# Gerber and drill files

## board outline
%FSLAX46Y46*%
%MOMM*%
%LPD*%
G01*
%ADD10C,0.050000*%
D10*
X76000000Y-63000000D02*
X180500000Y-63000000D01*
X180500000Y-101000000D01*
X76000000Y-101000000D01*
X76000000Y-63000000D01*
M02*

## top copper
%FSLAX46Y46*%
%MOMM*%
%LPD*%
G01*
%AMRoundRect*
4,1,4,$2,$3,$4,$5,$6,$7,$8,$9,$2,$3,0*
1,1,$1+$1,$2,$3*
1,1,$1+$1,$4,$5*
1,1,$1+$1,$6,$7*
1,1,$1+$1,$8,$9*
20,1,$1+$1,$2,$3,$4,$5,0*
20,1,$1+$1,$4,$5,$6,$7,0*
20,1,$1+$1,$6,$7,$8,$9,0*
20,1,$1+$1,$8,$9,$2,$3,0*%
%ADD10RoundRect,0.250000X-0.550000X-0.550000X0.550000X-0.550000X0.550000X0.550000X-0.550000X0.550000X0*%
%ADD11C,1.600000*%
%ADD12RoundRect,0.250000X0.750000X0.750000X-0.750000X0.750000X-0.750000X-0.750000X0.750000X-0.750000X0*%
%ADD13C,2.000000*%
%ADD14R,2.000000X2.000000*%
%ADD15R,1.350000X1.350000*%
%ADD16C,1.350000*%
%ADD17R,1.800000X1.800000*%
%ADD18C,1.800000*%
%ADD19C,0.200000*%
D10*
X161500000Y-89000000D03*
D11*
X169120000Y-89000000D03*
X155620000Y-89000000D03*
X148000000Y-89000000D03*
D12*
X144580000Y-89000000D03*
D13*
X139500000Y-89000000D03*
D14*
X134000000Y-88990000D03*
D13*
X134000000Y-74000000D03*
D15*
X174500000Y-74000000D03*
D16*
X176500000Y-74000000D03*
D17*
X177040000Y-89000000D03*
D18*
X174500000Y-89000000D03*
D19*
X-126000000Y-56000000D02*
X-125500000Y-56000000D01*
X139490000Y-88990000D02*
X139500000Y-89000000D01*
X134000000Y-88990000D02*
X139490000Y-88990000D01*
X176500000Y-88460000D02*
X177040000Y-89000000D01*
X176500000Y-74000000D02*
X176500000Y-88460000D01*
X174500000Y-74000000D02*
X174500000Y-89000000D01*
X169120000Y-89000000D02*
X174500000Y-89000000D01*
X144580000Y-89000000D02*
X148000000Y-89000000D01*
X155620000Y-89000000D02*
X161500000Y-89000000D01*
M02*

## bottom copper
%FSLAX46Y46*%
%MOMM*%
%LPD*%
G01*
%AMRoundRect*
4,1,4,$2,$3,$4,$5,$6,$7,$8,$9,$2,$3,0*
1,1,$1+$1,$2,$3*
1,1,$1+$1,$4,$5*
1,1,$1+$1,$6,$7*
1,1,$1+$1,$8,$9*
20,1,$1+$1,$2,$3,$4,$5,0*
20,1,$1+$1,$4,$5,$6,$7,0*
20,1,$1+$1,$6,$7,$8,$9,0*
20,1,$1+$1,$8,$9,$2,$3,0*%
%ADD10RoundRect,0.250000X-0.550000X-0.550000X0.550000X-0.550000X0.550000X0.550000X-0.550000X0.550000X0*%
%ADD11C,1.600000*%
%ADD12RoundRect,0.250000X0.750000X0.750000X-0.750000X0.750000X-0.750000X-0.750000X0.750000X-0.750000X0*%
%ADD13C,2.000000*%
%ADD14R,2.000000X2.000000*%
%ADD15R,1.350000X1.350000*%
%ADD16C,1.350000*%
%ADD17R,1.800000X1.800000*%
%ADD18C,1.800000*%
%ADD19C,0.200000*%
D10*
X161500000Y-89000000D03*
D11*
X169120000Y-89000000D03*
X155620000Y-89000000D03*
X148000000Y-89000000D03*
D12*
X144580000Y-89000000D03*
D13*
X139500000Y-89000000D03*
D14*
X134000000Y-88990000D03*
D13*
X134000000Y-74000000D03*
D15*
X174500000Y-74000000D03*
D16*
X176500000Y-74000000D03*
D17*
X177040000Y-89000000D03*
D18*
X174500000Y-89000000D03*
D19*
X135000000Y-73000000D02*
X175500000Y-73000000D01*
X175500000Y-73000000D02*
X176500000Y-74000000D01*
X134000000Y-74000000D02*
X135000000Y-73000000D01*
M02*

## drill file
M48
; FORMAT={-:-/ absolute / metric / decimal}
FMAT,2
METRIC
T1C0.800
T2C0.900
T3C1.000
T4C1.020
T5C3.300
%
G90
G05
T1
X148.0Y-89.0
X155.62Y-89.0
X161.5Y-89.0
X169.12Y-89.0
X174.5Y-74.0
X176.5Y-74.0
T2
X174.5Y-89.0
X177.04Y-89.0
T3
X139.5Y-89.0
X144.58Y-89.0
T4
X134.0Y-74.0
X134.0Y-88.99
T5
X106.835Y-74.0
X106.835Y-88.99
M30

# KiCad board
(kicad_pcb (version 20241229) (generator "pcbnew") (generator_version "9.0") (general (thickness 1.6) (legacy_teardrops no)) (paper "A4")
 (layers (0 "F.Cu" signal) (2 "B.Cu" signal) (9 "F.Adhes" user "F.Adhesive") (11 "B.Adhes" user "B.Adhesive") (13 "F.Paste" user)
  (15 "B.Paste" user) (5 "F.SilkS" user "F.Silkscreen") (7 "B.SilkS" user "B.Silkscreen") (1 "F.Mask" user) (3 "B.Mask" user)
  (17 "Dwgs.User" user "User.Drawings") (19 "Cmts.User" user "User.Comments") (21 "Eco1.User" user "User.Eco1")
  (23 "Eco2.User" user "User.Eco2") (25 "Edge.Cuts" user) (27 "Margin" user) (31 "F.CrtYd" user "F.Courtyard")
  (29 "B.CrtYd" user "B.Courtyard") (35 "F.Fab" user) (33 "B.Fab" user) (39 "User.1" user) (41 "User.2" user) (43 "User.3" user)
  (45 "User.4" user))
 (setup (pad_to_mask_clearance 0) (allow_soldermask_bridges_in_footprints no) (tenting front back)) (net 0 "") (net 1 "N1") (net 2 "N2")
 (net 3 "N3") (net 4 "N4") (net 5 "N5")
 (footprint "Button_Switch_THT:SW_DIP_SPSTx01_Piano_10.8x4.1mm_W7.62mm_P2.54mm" (layer "F.Cu") (at 161.5 89)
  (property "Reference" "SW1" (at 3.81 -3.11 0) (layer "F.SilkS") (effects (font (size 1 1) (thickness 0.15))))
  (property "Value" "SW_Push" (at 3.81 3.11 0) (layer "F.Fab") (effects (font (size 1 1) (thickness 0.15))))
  (pad "1" thru_hole roundrect (at 0 0) (size 1.6 1.6) (drill 0.8) (layers "*.Cu" "*.Mask") (remove_unused_layers no)
   (roundrect_rratio 0.15625) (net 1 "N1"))
  (pad "2" thru_hole circle (at 7.62 0) (size 1.6 1.6) (drill 0.8) (layers "*.Cu" "*.Mask") (remove_unused_layers no) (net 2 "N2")))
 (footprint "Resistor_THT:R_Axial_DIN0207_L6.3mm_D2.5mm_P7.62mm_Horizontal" (layer "F.Cu") (at 155.62 89 180)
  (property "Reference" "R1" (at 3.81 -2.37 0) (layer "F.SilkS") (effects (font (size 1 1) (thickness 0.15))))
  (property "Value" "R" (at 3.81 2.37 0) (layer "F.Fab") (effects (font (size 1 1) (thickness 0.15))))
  (pad "1" thru_hole circle (at 0 0 180) (size 1.6 1.6) (drill 0.8) (layers "*.Cu" "*.Mask") (remove_unused_layers no) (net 1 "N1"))
  (pad "2" thru_hole circle (at 7.62 0 180) (size 1.6 1.6) (drill 0.8) (layers "*.Cu" "*.Mask") (remove_unused_layers no) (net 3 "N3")))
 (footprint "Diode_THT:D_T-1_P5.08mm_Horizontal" (layer "F.Cu") (at 144.58 89 180)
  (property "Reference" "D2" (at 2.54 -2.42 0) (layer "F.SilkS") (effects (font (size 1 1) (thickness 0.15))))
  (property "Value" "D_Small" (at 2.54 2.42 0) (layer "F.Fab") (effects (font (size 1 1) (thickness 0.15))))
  (pad "1" thru_hole roundrect (at 0 0 180) (size 2 2) (drill 1) (layers "*.Cu" "*.Mask") (remove_unused_layers no) (roundrect_rratio 0.125)
   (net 3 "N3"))
  (pad "2" thru_hole circle (at 5.08 0 180) (size 2 2) (drill 1) (layers "*.Cu" "*.Mask") (remove_unused_layers no) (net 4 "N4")))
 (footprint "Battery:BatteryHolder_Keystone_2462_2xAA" (layer "F.Cu") (at 134 88.99 180)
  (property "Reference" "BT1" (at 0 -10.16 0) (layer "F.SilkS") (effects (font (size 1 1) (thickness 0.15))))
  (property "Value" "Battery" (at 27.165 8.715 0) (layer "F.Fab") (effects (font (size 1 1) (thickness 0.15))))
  (pad "" np_thru_hole circle (at 27.165 0 180) (size 3.3 3.3) (drill 3.3) (layers "*.Cu" "*.Mask"))
  (pad "" np_thru_hole circle (at 27.165 14.99 180) (size 3.3 3.3) (drill 3.3) (layers "*.Cu" "*.Mask"))
  (pad "1" thru_hole rect (at 0 0 180) (size 2 2) (drill 1.02) (layers "*.Cu" "*.Mask") (remove_unused_layers no) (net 4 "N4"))
  (pad "2" thru_hole circle (at 0 14.99 180) (size 2 2) (drill 1.02) (layers "*.Cu" "*.Mask") (remove_unused_layers no) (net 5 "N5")))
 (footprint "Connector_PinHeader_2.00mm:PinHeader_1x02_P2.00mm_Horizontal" (layer "F.Cu") (at 174.5 74 90)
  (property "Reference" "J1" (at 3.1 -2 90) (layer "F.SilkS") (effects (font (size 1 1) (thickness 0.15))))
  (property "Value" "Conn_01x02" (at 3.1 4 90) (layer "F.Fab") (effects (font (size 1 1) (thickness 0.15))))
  (pad "1" thru_hole rect (at 0 0 90) (size 1.35 1.35) (drill 0.8) (layers "*.Cu" "*.Mask") (remove_unused_layers no) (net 2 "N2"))
  (pad "2" thru_hole circle (at 0 2 90) (size 1.35 1.35) (drill 0.8) (layers "*.Cu" "*.Mask") (remove_unused_layers no) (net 5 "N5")))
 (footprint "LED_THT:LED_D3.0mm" (layer "F.Cu") (at 177.04 89 180)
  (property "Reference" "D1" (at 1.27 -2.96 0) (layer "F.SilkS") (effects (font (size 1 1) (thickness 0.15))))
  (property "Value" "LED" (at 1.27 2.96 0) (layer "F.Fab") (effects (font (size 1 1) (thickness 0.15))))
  (pad "1" thru_hole rect (at 0 0 180) (size 1.8 1.8) (drill 0.9) (layers "*.Cu" "*.Mask") (remove_unused_layers no) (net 5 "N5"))
  (pad "2" thru_hole circle (at 2.54 0 180) (size 1.8 1.8) (drill 0.9) (layers "*.Cu" "*.Mask") (remove_unused_layers no) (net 2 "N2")))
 (gr_rect (start 76 63) (end 180.5 101) (stroke (width 0.05) (type default)) (fill no) (layer "Edge.Cuts"))
 (segment (start -126 56) (end -125.5 56) (width 0.2) (layer "F.Cu") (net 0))
 (segment (start 139.49 88.99) (end 139.5 89) (width 0.2) (layer "F.Cu") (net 4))
 (segment (start 134 88.99) (end 139.49 88.99) (width 0.2) (layer "F.Cu") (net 4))
 (segment (start 176.5 88.46) (end 177.04 89) (width 0.2) (layer "F.Cu") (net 5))
 (segment (start 176.5 74) (end 176.5 88.46) (width 0.2) (layer "F.Cu") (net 5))
 (segment (start 135 73) (end 175.5 73) (width 0.2) (layer "B.Cu") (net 5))
 (segment (start 175.5 73) (end 176.5 74) (width 0.2) (layer "B.Cu") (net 5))
 (segment (start 134 74) (end 135 73) (width 0.2) (layer "B.Cu") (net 5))
 (segment (start 174.5 74) (end 174.5 89) (width 0.2) (layer "F.Cu") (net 2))
 (segment (start 169.12 89) (end 174.5 89) (width 0.2) (layer "F.Cu") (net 2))
 (segment (start 144.58 89) (end 148 89) (width 0.2) (layer "F.Cu") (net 3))
 (segment (start 155.62 89) (end 161.5 89) (width 0.2) (layer "F.Cu") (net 1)))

